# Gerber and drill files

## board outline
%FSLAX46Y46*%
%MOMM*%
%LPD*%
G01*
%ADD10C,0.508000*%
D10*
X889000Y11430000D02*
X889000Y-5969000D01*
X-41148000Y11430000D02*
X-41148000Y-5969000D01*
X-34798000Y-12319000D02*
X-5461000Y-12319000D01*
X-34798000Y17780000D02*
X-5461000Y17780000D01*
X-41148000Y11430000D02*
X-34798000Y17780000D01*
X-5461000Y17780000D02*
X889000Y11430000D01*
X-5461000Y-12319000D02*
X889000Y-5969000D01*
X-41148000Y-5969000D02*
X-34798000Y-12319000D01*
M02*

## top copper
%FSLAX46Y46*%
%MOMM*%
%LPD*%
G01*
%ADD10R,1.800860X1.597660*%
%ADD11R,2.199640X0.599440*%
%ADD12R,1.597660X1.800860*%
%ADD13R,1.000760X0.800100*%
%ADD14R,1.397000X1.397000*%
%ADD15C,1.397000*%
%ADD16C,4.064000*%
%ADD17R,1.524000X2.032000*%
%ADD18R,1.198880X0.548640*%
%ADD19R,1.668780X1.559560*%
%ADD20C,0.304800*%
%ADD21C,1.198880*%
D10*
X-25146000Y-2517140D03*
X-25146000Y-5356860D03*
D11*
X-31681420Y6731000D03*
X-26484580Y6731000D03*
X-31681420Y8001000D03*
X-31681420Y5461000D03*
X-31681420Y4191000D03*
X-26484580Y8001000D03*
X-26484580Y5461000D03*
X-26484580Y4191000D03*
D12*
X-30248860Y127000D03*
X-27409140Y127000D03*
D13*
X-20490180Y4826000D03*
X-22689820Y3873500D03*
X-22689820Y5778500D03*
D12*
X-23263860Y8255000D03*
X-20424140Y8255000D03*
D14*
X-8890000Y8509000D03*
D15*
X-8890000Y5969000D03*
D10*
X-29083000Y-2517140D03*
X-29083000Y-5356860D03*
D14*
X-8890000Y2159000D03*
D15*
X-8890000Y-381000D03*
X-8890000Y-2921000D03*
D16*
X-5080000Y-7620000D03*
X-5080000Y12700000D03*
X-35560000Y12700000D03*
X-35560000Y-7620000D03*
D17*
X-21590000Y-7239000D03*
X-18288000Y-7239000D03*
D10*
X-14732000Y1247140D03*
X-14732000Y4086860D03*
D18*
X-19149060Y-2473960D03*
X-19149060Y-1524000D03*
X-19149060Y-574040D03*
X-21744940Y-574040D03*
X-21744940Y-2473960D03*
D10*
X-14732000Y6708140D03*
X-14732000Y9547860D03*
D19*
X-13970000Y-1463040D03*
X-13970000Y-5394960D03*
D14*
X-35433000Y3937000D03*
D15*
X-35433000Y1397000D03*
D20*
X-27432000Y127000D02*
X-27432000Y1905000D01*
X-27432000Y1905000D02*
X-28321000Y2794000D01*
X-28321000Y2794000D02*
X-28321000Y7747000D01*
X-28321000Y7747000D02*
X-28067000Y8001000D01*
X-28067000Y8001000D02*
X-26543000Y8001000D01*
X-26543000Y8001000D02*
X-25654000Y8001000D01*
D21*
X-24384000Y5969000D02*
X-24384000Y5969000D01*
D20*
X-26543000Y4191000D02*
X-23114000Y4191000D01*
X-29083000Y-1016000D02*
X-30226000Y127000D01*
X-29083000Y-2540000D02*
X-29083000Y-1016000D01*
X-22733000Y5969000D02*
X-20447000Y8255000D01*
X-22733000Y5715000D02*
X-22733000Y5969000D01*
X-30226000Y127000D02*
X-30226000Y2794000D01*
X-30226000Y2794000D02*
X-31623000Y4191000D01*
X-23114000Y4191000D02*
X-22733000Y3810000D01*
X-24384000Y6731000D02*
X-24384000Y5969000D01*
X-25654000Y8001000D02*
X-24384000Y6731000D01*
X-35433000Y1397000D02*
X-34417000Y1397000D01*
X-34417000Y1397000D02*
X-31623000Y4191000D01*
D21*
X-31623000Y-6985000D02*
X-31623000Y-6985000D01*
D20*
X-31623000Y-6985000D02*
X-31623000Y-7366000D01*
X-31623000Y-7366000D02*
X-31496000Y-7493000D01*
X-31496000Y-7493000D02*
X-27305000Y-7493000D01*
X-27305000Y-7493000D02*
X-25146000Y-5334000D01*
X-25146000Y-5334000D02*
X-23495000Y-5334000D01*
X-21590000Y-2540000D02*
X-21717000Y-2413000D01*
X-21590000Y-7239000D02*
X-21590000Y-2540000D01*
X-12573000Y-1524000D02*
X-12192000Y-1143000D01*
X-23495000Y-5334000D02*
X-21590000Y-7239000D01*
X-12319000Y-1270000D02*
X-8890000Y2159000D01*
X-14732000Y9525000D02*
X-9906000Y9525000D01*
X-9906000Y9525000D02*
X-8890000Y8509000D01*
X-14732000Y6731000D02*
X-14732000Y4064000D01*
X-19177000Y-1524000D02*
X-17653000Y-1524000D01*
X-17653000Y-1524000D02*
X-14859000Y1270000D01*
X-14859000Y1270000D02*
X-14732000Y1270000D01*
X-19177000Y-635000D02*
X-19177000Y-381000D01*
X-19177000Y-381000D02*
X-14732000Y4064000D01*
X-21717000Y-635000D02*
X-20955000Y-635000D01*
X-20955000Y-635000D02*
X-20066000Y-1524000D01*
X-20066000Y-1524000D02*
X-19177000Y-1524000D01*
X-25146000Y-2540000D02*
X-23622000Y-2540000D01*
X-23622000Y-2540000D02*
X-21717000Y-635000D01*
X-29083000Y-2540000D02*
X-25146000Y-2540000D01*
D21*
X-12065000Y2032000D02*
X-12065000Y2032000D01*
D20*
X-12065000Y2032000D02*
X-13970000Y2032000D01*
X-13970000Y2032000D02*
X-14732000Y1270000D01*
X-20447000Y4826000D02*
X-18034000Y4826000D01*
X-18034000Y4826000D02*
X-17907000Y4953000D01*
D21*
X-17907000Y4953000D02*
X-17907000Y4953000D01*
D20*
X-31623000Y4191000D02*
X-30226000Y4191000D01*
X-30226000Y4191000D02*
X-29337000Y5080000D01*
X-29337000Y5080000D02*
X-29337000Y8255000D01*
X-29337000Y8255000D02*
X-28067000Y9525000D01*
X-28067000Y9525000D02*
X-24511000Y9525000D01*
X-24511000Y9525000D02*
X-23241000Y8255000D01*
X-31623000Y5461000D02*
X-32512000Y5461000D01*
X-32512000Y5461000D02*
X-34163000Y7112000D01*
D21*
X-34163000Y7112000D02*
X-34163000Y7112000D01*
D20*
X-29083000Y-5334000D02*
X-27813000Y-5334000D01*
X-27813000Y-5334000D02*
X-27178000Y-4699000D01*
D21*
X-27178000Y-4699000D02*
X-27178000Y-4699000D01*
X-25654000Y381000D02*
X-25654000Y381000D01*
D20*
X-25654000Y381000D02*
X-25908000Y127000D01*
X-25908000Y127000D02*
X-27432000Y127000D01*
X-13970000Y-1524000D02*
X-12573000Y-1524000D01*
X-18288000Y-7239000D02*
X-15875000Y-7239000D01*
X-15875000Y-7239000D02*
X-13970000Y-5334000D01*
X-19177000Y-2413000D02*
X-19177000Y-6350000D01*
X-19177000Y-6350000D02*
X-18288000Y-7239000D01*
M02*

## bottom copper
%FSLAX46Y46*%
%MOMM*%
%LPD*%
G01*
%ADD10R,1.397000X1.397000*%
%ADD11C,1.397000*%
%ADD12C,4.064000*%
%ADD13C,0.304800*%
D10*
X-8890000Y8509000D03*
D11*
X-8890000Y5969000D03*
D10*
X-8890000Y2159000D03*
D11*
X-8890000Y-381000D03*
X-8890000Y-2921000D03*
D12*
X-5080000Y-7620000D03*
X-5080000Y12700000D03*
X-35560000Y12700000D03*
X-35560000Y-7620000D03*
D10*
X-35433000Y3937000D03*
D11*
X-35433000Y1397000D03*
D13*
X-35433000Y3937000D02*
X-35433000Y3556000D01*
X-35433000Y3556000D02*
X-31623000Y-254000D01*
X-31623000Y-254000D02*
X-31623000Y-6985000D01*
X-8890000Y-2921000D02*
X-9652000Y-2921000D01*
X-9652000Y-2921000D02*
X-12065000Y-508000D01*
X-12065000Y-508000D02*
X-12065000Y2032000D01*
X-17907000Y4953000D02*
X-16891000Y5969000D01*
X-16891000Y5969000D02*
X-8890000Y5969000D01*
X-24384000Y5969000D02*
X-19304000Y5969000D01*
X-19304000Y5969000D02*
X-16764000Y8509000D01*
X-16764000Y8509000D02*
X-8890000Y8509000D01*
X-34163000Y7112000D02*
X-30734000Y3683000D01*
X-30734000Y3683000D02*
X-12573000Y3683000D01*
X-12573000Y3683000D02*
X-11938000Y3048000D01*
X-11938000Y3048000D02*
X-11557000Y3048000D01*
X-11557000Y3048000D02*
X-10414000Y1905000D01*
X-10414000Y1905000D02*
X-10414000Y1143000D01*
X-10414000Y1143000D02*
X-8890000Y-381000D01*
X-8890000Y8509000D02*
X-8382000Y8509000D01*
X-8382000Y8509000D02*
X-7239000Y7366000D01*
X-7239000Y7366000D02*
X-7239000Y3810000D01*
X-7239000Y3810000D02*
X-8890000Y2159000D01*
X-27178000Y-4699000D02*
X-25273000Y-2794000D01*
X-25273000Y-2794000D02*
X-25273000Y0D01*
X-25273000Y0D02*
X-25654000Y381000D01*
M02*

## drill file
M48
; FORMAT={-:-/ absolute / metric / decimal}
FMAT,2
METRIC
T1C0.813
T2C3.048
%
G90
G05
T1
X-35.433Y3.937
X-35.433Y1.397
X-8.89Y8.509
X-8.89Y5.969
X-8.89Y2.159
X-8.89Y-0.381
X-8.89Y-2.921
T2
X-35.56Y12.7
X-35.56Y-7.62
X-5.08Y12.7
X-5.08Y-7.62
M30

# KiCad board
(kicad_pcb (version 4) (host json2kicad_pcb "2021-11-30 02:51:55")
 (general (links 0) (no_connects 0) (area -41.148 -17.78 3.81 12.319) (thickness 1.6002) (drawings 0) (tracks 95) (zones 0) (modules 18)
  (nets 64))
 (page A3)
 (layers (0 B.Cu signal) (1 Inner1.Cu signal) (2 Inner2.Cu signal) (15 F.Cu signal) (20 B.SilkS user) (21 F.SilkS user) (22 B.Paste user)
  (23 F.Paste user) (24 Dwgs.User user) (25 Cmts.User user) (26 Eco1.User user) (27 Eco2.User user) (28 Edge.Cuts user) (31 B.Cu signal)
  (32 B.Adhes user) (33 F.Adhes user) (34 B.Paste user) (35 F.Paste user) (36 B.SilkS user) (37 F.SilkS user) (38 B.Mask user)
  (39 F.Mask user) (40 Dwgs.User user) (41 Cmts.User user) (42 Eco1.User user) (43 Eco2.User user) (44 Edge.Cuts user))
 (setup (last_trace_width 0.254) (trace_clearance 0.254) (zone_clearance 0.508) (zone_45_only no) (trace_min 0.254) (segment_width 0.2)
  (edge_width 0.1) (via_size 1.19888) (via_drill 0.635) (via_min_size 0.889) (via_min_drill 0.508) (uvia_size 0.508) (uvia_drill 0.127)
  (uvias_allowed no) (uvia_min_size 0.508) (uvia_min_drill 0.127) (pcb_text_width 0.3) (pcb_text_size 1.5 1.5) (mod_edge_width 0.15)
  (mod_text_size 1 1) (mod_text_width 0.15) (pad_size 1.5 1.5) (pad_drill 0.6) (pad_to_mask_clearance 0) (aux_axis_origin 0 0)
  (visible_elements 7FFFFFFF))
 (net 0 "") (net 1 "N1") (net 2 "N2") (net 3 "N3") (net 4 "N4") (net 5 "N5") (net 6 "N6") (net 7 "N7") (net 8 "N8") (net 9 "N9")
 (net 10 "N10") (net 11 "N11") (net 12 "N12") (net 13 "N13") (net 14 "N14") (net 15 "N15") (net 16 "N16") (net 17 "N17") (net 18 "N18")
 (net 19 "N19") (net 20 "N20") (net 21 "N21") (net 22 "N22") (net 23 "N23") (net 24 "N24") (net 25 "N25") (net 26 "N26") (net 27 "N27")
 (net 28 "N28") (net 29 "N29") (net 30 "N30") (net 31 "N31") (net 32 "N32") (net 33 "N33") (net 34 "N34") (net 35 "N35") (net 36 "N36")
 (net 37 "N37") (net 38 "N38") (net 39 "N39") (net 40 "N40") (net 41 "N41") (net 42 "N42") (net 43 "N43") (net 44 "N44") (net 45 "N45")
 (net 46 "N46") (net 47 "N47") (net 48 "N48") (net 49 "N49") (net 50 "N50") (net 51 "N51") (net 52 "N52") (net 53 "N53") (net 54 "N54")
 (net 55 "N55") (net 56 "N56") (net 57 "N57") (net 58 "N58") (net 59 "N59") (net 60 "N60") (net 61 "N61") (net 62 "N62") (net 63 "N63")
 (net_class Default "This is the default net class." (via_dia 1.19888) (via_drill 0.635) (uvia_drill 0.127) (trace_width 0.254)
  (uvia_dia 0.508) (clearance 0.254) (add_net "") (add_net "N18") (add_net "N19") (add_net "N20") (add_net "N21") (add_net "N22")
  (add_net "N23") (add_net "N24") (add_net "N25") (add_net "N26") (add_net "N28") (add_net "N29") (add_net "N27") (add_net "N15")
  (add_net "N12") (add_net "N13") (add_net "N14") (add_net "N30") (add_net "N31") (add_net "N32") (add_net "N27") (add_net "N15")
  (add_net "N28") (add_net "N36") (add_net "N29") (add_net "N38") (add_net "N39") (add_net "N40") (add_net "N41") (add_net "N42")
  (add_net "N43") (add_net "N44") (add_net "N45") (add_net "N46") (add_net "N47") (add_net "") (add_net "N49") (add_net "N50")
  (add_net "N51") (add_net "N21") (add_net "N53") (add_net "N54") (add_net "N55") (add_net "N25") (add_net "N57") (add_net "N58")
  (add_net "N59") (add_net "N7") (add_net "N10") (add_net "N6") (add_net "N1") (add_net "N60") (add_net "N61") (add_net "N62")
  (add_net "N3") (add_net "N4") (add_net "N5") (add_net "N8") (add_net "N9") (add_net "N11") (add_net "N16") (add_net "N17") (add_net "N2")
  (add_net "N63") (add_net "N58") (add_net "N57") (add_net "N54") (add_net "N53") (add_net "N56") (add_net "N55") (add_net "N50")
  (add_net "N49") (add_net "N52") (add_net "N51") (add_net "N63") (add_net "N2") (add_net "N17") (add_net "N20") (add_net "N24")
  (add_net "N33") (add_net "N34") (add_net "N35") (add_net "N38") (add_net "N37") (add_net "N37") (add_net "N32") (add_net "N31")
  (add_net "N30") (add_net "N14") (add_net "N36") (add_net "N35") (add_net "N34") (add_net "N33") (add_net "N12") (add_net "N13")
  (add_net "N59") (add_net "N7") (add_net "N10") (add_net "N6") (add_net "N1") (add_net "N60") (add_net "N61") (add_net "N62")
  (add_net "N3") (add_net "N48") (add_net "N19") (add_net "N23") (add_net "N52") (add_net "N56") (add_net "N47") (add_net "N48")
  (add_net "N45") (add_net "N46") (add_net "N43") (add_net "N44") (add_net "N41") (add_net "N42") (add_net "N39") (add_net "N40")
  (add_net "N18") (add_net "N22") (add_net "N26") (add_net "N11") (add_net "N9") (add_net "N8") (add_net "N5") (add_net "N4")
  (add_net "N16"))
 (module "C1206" (layer "F.Cu") (at -25.146 3.937 90.00)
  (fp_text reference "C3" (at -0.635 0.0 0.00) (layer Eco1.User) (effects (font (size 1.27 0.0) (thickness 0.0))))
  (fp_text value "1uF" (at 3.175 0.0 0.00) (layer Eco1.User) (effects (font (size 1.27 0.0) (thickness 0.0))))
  (pad 2 smd rect (at 1.41986 0.0 90.00) (size 1.59766 1.80086) (drill 0.0) (layers "F.Cu" "F.Paste") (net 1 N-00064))
  (pad 1 smd rect (at -1.41986 0.0 90.00) (size 1.59766 1.80086) (drill 0.0) (layers "F.Cu" "F.Paste") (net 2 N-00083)))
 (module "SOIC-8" (layer "F.Cu") (at -29.083 -6.096 -90.00)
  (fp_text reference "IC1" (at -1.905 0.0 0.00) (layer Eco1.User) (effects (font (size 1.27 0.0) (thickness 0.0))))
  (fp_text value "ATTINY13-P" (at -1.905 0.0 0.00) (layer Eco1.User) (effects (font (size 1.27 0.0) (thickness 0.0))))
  (pad 2 smd rect (at -0.635 2.59842 -90.00) (size 0.59944 2.19964) (drill 0.0) (layers "F.Cu" "F.Paste") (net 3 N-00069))
  (pad 7 smd rect (at -0.635 -2.59842 -90.00) (size 0.59944 2.19964) (drill 0.0) (layers "F.Cu" "F.Paste") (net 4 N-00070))
  (pad 1 smd rect (at -1.905 2.59842 -90.00) (size 0.59944 2.19964) (drill 0.0) (layers "F.Cu" "F.Paste") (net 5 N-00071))
  (pad 3 smd rect (at 0.635 2.59842 -90.00) (size 0.59944 2.19964) (drill 0.0) (layers "F.Cu" "F.Paste") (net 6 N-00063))
  (pad 4 smd rect (at 1.905 2.59842 -90.00) (size 0.59944 2.19964) (drill 0.0) (layers "F.Cu" "F.Paste") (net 1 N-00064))
  (pad 8 smd rect (at -1.905 -2.59842 -90.00) (size 0.59944 2.19964) (drill 0.0) (layers "F.Cu" "F.Paste") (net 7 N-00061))
  (pad 6 smd rect (at 0.635 -2.59842 -90.00) (size 0.59944 2.19964) (drill 0.0) (layers "F.Cu" "F.Paste") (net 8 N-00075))
  (pad 5 smd rect (at 1.905 -2.59842 -90.00) (size 0.59944 2.19964) (drill 0.0) (layers "F.Cu" "F.Paste") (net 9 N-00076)))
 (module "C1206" (layer "F.Cu") (at -28.829 -0.127 -180.00)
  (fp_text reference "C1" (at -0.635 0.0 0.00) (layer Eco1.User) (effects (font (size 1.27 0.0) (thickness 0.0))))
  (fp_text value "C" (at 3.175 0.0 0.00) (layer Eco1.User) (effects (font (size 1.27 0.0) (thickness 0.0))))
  (pad 2 smd rect (at 1.41986 0.0 -180.00) (size 1.59766 1.80086) (drill 0.0) (layers "F.Cu" "F.Paste") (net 1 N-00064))
  (pad 1 smd rect (at -1.41986 0.0 -180.00) (size 1.59766 1.80086) (drill 0.0) (layers "F.Cu" "F.Paste") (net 7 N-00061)))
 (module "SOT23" (layer "F.Cu") (at -21.59 -4.826 -90.00)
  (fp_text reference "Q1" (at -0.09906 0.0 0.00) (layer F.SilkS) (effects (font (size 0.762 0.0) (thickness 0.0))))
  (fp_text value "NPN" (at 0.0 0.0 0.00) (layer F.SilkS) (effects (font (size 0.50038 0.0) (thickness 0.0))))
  (pad 3 smd rect (at 0.0 -1.09982 -90.00) (size 0.8001 1.00076) (drill 0.0) (layers "F.Cu" "F.Paste") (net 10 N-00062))
  (pad 2 smd rect (at 0.9525 1.09982 -90.00) (size 0.8001 1.00076) (drill 0.0) (layers "F.Cu" "F.Paste") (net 9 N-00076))
  (pad 1 smd rect (at -0.9525 1.09982 -90.00) (size 0.8001 1.00076) (drill 0.0) (layers "F.Cu" "F.Paste") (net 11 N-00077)))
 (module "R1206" (layer "F.Cu") (at -21.844 -8.255 -180.00)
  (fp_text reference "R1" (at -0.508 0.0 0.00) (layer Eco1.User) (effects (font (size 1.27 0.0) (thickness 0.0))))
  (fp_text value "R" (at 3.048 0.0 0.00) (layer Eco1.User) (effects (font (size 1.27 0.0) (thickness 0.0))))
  (pad 2 smd rect (at 1.41986 0.0 -180.00) (size 1.59766 1.80086) (drill 0.0) (layers "F.Cu" "F.Paste") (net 1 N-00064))
  (pad 1 smd rect (at -1.41986 0.0 -180.00) (size 1.59766 1.80086) (drill 0.0) (layers "F.Cu" "F.Paste") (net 11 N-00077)))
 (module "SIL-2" (layer "F.Cu") (at -8.89 -7.239 -90.00)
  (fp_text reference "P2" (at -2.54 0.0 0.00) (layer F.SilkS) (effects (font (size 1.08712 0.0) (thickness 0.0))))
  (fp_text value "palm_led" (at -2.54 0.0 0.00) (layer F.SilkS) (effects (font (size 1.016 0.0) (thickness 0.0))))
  (pad 1 thru_hole rect (at -1.27 0.0 -90.00) (size 1.397 1.397) (drill 0.8128)
   (layers "B.Cu" "Inner1.Cu" "Inner2.Cu" "F.Cu" "F.SilkS" "B.Paste" "F.Paste") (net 7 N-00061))
  (pad 2 thru_hole circle (at 1.27 0.0 -90.00) (size 1.397 1.397) (drill 0.8128)
   (layers "B.Cu" "Inner1.Cu" "Inner2.Cu" "F.Cu" "F.SilkS" "B.Paste" "F.Paste") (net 10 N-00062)))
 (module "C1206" (layer "F.Cu") (at -29.083 3.937 90.00)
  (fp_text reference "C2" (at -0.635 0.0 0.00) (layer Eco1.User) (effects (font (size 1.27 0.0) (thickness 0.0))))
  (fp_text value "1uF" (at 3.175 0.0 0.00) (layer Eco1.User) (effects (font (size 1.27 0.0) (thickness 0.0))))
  (pad 2 smd rect (at 1.41986 0.0 90.00) (size 1.59766 1.80086) (drill 0.0) (layers "F.Cu" "F.Paste") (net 1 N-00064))
  (pad 1 smd rect (at -1.41986 0.0 90.00) (size 1.59766 1.80086) (drill 0.0) (layers "F.Cu" "F.Paste") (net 7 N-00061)))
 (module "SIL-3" (layer "F.Cu") (at -8.89 0.381 -90.00)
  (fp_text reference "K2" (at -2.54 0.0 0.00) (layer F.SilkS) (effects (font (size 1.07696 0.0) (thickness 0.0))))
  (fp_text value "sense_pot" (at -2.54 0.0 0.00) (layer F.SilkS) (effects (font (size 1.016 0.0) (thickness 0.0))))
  (pad 1 thru_hole rect (at -2.54 0.0 -90.00) (size 1.397 1.397) (drill 0.8128)
   (layers "B.Cu" "Inner1.Cu" "Inner2.Cu" "F.Cu" "F.SilkS" "B.Paste" "F.Paste") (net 7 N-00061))
  (pad 2 thru_hole circle (at 0.0 0.0 -90.00) (size 1.397 1.397) (drill 0.8128)
   (layers "B.Cu" "Inner1.Cu" "Inner2.Cu" "F.Cu" "F.SilkS" "B.Paste" "F.Paste") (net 6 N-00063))
  (pad 3 thru_hole circle (at 2.54 0.0 -90.00) (size 1.397 1.397) (drill 0.8128)
   (layers "B.Cu" "Inner1.Cu" "Inner2.Cu" "F.Cu" "F.SilkS" "B.Paste" "F.Paste") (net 1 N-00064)))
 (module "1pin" (layer "F.Cu") (at -5.08 7.62 0.00)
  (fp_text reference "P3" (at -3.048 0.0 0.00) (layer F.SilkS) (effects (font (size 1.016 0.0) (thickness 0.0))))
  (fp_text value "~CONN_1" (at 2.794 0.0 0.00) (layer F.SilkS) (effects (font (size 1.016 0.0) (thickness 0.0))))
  (pad 1 thru_hole circle (at 0.0 0.0 0.00) (size 4.064 4.064) (drill 3.048)
   (layers "B.Cu" "Inner1.Cu" "Inner2.Cu" "F.Cu" "F.SilkS" "B.Paste" "F.Paste") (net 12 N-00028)))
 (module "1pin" (layer "F.Cu") (at -5.08 -12.7 0.00)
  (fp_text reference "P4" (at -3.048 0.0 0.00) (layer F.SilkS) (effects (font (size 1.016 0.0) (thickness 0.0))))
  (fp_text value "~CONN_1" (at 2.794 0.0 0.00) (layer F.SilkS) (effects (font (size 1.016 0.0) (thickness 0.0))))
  (pad 1 thru_hole circle (at 0.0 0.0 0.00) (size 4.064 4.064) (drill 3.048)
   (layers "B.Cu" "Inner1.Cu" "Inner2.Cu" "F.Cu" "F.SilkS" "B.Paste" "F.Paste") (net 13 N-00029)))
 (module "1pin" (layer "F.Cu") (at -35.56 -12.7 0.00)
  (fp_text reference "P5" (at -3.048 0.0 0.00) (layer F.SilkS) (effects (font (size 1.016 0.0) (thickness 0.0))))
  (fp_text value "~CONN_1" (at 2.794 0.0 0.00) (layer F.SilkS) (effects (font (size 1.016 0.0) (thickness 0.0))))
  (pad 1 thru_hole circle (at 0.0 0.0 0.00) (size 4.064 4.064) (drill 3.048)
   (layers "B.Cu" "Inner1.Cu" "Inner2.Cu" "F.Cu" "F.SilkS" "B.Paste" "F.Paste") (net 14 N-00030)))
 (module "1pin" (layer "F.Cu") (at -35.56 7.62 0.00)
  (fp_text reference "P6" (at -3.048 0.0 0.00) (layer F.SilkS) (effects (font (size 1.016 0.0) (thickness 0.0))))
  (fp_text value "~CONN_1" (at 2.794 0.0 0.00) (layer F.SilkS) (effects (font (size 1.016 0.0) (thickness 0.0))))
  (pad 1 thru_hole circle (at 0.0 0.0 0.00) (size 4.064 4.064) (drill 3.048)
   (layers "B.Cu" "Inner1.Cu" "Inner2.Cu" "F.Cu" "F.SilkS" "B.Paste" "F.Paste") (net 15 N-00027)))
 (segment (start -27.432 -0.127) (end -27.432 -1.905) (width 0.3048) (layer F.Cu) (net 7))
 (segment (start -27.432 -1.905) (end -28.321 -2.794) (width 0.3048) (layer F.Cu) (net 7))
 (segment (start -28.321 -2.794) (end -28.321 -7.747) (width 0.3048) (layer F.Cu) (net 7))
 (segment (start -28.321 -7.747) (end -28.067 -8.001) (width 0.3048) (layer F.Cu) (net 7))
 (segment (start -28.067 -8.001) (end -26.543 -8.001) (width 0.3048) (layer F.Cu) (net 7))
 (segment (start -26.543 -8.001) (end -25.654 -8.001) (width 0.3048) (layer F.Cu) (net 7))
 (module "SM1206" (layer "F.Cu") (at -19.939 7.239 0.00)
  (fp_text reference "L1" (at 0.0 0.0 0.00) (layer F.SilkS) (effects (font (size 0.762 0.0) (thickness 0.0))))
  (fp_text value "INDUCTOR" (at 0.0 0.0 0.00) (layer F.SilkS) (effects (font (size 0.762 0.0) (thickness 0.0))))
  (pad 1 smd rect (at -1.651 0.0 0.00) (size 1.524 2.032) (drill 0.0) (layers "F.Cu" "F.Paste") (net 2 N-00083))
  (pad 2 smd rect (at 1.651 0.0 0.00) (size 1.524 2.032) (drill 0.0) (layers "F.Cu" "F.Paste") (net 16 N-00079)))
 (segment (start -24.384 -5.969) (end -24.384 -5.969) (width 1.19888) (layer F.Cu) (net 7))
 (segment (start -26.543 -4.191) (end -23.114 -4.191) (width 0.3048) (layer F.Cu) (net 9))
 (segment (start -29.083 1.016) (end -30.226 -0.127) (width 0.3048) (layer F.Cu) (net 1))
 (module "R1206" (layer "F.Cu") (at -14.732 -2.667 -90.00)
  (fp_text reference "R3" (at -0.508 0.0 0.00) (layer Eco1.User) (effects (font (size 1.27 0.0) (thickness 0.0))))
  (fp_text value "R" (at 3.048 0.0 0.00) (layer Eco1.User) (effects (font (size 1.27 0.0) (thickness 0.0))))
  (pad 2 smd rect (at 1.41986 0.0 -90.00) (size 1.59766 1.80086) (drill 0.0) (layers "F.Cu" "F.Paste") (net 1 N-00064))
  (pad 1 smd rect (at -1.41986 0.0 -90.00) (size 1.59766 1.80086) (drill 0.0) (layers "F.Cu" "F.Paste") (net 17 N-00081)))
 (segment (start -29.083 2.54) (end -29.083 1.016) (width 0.3048) (layer F.Cu) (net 1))
 (segment (start -22.733 -5.969) (end -20.447 -8.255) (width 0.3048) (layer F.Cu) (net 11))
 (segment (start -22.733 -5.715) (end -22.733 -5.969) (width 0.3048) (layer F.Cu) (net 11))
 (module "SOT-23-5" (layer "F.Cu") (at -20.447 1.524 90.00)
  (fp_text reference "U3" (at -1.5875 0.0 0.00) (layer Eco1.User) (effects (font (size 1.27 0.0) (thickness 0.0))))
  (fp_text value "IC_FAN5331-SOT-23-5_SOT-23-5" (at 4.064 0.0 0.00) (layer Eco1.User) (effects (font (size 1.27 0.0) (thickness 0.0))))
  (pad 1 smd rect (at -0.94996 1.29794 90.00) (size 0.54864 1.19888) (drill 0.0) (layers "F.Cu" "F.Paste") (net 16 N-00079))
  (pad 2 smd rect (at 0.0 1.29794 90.00) (size 0.54864 1.19888) (drill 0.0) (layers "F.Cu" "F.Paste") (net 1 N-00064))
  (pad 3 smd rect (at 0.94996 1.29794 90.00) (size 0.54864 1.19888) (drill 0.0) (layers "F.Cu" "F.Paste") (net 17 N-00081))
  (pad 4 smd rect (at 0.94996 -1.29794 90.00) (size 0.54864 1.19888) (drill 0.0) (layers "F.Cu" "F.Paste") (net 1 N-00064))
  (pad 5 smd rect (at -0.94996 -1.29794 90.00) (size 0.54864 1.19888) (drill 0.0) (layers "F.Cu" "F.Paste") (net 2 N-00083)))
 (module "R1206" (layer "F.Cu") (at -14.732 -8.128 -90.00)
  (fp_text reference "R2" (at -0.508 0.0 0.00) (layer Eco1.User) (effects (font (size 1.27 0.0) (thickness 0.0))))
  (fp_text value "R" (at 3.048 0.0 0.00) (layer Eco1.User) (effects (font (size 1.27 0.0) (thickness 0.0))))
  (pad 2 smd rect (at 1.41986 0.0 -90.00) (size 1.59766 1.80086) (drill 0.0) (layers "F.Cu" "F.Paste") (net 17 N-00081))
  (pad 1 smd rect (at -1.41986 0.0 -90.00) (size 1.59766 1.80086) (drill 0.0) (layers "F.Cu" "F.Paste") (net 7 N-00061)))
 (segment (start -30.226 -0.127) (end -30.226 -2.794) (width 0.3048) (layer F.Cu) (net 1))
 (segment (start -30.226 -2.794) (end -31.623 -4.191) (width 0.3048) (layer F.Cu) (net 1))
 (segment (start -23.114 -4.191) (end -22.733 -3.81) (width 0.3048) (layer F.Cu) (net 9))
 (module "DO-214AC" (layer "F.Cu") (at -13.97 3.429 90.00)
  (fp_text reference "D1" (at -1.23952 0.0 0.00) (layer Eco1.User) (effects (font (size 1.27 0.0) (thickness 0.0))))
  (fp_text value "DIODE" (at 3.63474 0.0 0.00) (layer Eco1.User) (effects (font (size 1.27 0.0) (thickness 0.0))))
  (pad 2 smd rect (at 1.96596 0.0 90.00) (size 1.55956 1.66878) (drill 0.0) (layers "F.Cu" "F.Paste") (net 7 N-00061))
  (pad 1 smd rect (at -1.96596 0.0 90.00) (size 1.55956 1.66878) (drill 0.0) (layers "F.Cu" "F.Paste") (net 16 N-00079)))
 (segment (start -24.384 -6.731) (end -24.384 -5.969) (width 0.3048) (layer F.Cu) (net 7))
 (segment (start -25.654 -8.001) (end -24.384 -6.731) (width 0.3048) (layer F.Cu) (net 7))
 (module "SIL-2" (layer "F.Cu") (at -35.433 -2.667 -90.00)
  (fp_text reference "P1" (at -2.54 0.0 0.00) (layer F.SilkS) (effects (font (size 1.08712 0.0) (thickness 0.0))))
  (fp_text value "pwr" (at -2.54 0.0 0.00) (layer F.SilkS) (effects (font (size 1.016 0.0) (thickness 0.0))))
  (pad 1 thru_hole rect (at -1.27 0.0 -90.00) (size 1.397 1.397) (drill 0.8128)
   (layers "B.Cu" "Inner1.Cu" "Inner2.Cu" "F.Cu" "F.SilkS" "B.Paste" "F.Paste") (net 2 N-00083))
  (pad 2 thru_hole circle (at 1.27 0.0 -90.00) (size 1.397 1.397) (drill 0.8128)
   (layers "B.Cu" "Inner1.Cu" "Inner2.Cu" "F.Cu" "F.SilkS" "B.Paste" "F.Paste") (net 1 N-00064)))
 (segment (start -35.433 -1.397) (end -34.417 -1.397) (width 0.3048) (layer F.Cu) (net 1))
 (segment (start -34.417 -1.397) (end -31.623 -4.191) (width 0.3048) (layer F.Cu) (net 1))
 (segment (start -35.433 -3.937) (end -35.433 -3.556) (width 0.3048) (layer B.Cu) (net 2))
 (segment (start -35.433 -3.556) (end -31.623 0.254) (width 0.3048) (layer B.Cu) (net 2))
 (segment (start -31.623 0.254) (end -31.623 6.985) (width 0.3048) (layer B.Cu) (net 2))
 (segment (start -31.623 6.985) (end -31.623 6.985) (width 1.19888) (layer F.Cu) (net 2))
 (segment (start -31.623 6.985) (end -31.623 7.366) (width 0.3048) (layer F.Cu) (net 2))
 (segment (start -31.623 7.366) (end -31.496 7.493) (width 0.3048) (layer F.Cu) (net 2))
 (segment (start -31.496 7.493) (end -27.305 7.493) (width 0.3048) (layer F.Cu) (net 2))
 (segment (start -27.305 7.493) (end -25.146 5.334) (width 0.3048) (layer F.Cu) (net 2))
 (segment (start -25.146 5.334) (end -23.495 5.334) (width 0.3048) (layer F.Cu) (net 2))
 (segment (start -21.59 2.54) (end -21.717 2.413) (width 0.3048) (layer F.Cu) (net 2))
 (segment (start -21.59 7.239) (end -21.59 2.54) (width 0.3048) (layer F.Cu) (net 2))
 (gr_line (start 0.889 -11.43) (end 0.889 5.969) (angle 51566.20) (width 0.508) (layer Edge.Cuts))
 (segment (start -12.573 1.524) (end -12.192 1.143) (width 0.3048) (layer F.Cu) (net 7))
 (segment (start -23.495 5.334) (end -21.59 7.239) (width 0.3048) (layer F.Cu) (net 2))
 (gr_line (start -41.148 -11.43) (end -41.148 5.969) (angle 51566.20) (width 0.508) (layer Edge.Cuts))
 (gr_line (start -34.798 12.319) (end -5.461 12.319) (angle 51566.20) (width 0.508) (layer Edge.Cuts))
 (segment (start -12.319 1.27) (end -8.89 -2.159) (width 0.3048) (layer F.Cu) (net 7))
 (segment (start -14.732 -9.525) (end -9.906 -9.525) (width 0.3048) (layer F.Cu) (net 7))
 (segment (start -9.906 -9.525) (end -8.89 -8.509) (width 0.3048) (layer F.Cu) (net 7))
 (segment (start -14.732 -6.731) (end -14.732 -4.064) (width 0.3048) (layer F.Cu) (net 17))
 (segment (start -19.177 1.524) (end -17.653 1.524) (width 0.3048) (layer F.Cu) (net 1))
 (segment (start -17.653 1.524) (end -14.859 -1.27) (width 0.3048) (layer F.Cu) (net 1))
 (segment (start -14.859 -1.27) (end -14.732 -1.27) (width 0.3048) (layer F.Cu) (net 1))
 (segment (start -19.177 0.635) (end -19.177 0.381) (width 0.3048) (layer F.Cu) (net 17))
 (segment (start -19.177 0.381) (end -14.732 -4.064) (width 0.3048) (layer F.Cu) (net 17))
 (segment (start -21.717 0.635) (end -20.955 0.635) (width 0.3048) (layer F.Cu) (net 1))
 (segment (start -20.955 0.635) (end -20.066 1.524) (width 0.3048) (layer F.Cu) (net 1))
 (segment (start -20.066 1.524) (end -19.177 1.524) (width 0.3048) (layer F.Cu) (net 1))
 (segment (start -25.146 2.54) (end -23.622 2.54) (width 0.3048) (layer F.Cu) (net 1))
 (segment (start -23.622 2.54) (end -21.717 0.635) (width 0.3048) (layer F.Cu) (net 1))
 (segment (start -29.083 2.54) (end -25.146 2.54) (width 0.3048) (layer F.Cu) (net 1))
 (segment (start -8.89 2.921) (end -9.652 2.921) (width 0.3048) (layer B.Cu) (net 1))
 (segment (start -9.652 2.921) (end -12.065 0.508) (width 0.3048) (layer B.Cu) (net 1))
 (segment (start -12.065 0.508) (end -12.065 -2.032) (width 0.3048) (layer B.Cu) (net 1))
 (segment (start -12.065 -2.032) (end -12.065 -2.032) (width 1.19888) (layer F.Cu) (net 1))
 (segment (start -12.065 -2.032) (end -13.97 -2.032) (width 0.3048) (layer F.Cu) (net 1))
 (segment (start -13.97 -2.032) (end -14.732 -1.27) (width 0.3048) (layer F.Cu) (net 1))
 (segment (start -20.447 -4.826) (end -18.034 -4.826) (width 0.3048) (layer F.Cu) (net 10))
 (segment (start -18.034 -4.826) (end -17.907 -4.953) (width 0.3048) (layer F.Cu) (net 10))
 (segment (start -17.907 -4.953) (end -17.907 -4.953) (width 1.19888) (layer F.Cu) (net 10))
 (segment (start -17.907 -4.953) (end -16.891 -5.969) (width 0.3048) (layer B.Cu) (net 10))
 (segment (start -16.891 -5.969) (end -8.89 -5.969) (width 0.3048) (layer B.Cu) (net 10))
 (segment (start -24.384 -5.969) (end -19.304 -5.969) (width 0.3048) (layer B.Cu) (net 7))
 (segment (start -19.304 -5.969) (end -16.764 -8.509) (width 0.3048) (layer B.Cu) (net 7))
 (segment (start -16.764 -8.509) (end -8.89 -8.509) (width 0.3048) (layer B.Cu) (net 7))
 (segment (start -31.623 -4.191) (end -30.226 -4.191) (width 0.3048) (layer F.Cu) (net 1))
 (segment (start -30.226 -4.191) (end -29.337 -5.08) (width 0.3048) (layer F.Cu) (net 1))
 (segment (start -29.337 -5.08) (end -29.337 -8.255) (width 0.3048) (layer F.Cu) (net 1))
 (segment (start -29.337 -8.255) (end -28.067 -9.525) (width 0.3048) (layer F.Cu) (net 1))
 (segment (start -28.067 -9.525) (end -24.511 -9.525) (width 0.3048) (layer F.Cu) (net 1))
 (segment (start -24.511 -9.525) (end -23.241 -8.255) (width 0.3048) (layer F.Cu) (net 1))
 (segment (start -31.623 -5.461) (end -32.512 -5.461) (width 0.3048) (layer F.Cu) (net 6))
 (segment (start -32.512 -5.461) (end -34.163 -7.112) (width 0.3048) (layer F.Cu) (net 6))
 (segment (start -34.163 -7.112) (end -34.163 -7.112) (width 1.19888) (layer F.Cu) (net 6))
 (segment (start -34.163 -7.112) (end -30.734 -3.683) (width 0.3048) (layer B.Cu) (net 6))
 (segment (start -30.734 -3.683) (end -12.573 -3.683) (width 0.3048) (layer B.Cu) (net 6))
 (segment (start -12.573 -3.683) (end -11.938 -3.048) (width 0.3048) (layer B.Cu) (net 6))
 (segment (start -11.938 -3.048) (end -11.557 -3.048) (width 0.3048) (layer B.Cu) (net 6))
 (segment (start -11.557 -3.048) (end -10.414 -1.905) (width 0.3048) (layer B.Cu) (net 6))
 (segment (start -10.414 -1.905) (end -10.414 -1.143) (width 0.3048) (layer B.Cu) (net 6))
 (segment (start -10.414 -1.143) (end -8.89 0.381) (width 0.3048) (layer B.Cu) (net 6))
 (segment (start -8.89 -8.509) (end -8.382 -8.509) (width 0.3048) (layer B.Cu) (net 7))
 (segment (start -8.382 -8.509) (end -7.239 -7.366) (width 0.3048) (layer B.Cu) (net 7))
 (segment (start -7.239 -7.366) (end -7.239 -3.81) (width 0.3048) (layer B.Cu) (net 7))
 (segment (start -7.239 -3.81) (end -8.89 -2.159) (width 0.3048) (layer B.Cu) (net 7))
 (segment (start -29.083 5.334) (end -27.813 5.334) (width 0.3048) (layer F.Cu) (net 7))
 (segment (start -27.813 5.334) (end -27.178 4.699) (width 0.3048) (layer F.Cu) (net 7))
 (segment (start -27.178 4.699) (end -27.178 4.699) (width 1.19888) (layer F.Cu) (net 7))
 (segment (start -27.178 4.699) (end -25.273 2.794) (width 0.3048) (layer B.Cu) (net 7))
 (segment (start -25.273 2.794) (end -25.273 0.0) (width 0.3048) (layer B.Cu) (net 7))
 (segment (start -25.273 0.0) (end -25.654 -0.381) (width 0.3048) (layer B.Cu) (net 7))
 (segment (start -25.654 -0.381) (end -25.654 -0.381) (width 1.19888) (layer F.Cu) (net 7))
 (segment (start -25.654 -0.381) (end -25.908 -0.127) (width 0.3048) (layer F.Cu) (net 7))
 (segment (start -25.908 -0.127) (end -27.432 -0.127) (width 0.3048) (layer F.Cu) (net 7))
 (gr_line (start -34.798 -17.78) (end -5.461 -17.78) (angle 51566.20) (width 0.508) (layer Edge.Cuts))
 (segment (start -13.97 1.524) (end -12.573 1.524) (width 0.3048) (layer F.Cu) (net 7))
 (segment (start -18.288 7.239) (end -15.875 7.239) (width 0.3048) (layer F.Cu) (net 16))
 (segment (start -15.875 7.239) (end -13.97 5.334) (width 0.3048) (layer F.Cu) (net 16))
 (segment (start -19.177 2.413) (end -19.177 6.35) (width 0.3048) (layer F.Cu) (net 16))
 (segment (start -19.177 6.35) (end -18.288 7.239) (width 0.3048) (layer F.Cu) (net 16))
 (gr_line (start -41.148 -11.43) (end -34.798 -17.78) (angle 51566.20) (width 0.508) (layer Edge.Cuts))
 (gr_line (start -5.461 -17.78) (end 0.889 -11.43) (angle 51566.20) (width 0.508) (layer Edge.Cuts))
 (gr_line (start -5.461 12.319) (end 0.889 5.969) (angle 51566.20) (width 0.508) (layer Edge.Cuts))
 (gr_line (start -41.148 5.969) (end -34.798 12.319) (angle 51566.20) (width 0.508) (layer Edge.Cuts)))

